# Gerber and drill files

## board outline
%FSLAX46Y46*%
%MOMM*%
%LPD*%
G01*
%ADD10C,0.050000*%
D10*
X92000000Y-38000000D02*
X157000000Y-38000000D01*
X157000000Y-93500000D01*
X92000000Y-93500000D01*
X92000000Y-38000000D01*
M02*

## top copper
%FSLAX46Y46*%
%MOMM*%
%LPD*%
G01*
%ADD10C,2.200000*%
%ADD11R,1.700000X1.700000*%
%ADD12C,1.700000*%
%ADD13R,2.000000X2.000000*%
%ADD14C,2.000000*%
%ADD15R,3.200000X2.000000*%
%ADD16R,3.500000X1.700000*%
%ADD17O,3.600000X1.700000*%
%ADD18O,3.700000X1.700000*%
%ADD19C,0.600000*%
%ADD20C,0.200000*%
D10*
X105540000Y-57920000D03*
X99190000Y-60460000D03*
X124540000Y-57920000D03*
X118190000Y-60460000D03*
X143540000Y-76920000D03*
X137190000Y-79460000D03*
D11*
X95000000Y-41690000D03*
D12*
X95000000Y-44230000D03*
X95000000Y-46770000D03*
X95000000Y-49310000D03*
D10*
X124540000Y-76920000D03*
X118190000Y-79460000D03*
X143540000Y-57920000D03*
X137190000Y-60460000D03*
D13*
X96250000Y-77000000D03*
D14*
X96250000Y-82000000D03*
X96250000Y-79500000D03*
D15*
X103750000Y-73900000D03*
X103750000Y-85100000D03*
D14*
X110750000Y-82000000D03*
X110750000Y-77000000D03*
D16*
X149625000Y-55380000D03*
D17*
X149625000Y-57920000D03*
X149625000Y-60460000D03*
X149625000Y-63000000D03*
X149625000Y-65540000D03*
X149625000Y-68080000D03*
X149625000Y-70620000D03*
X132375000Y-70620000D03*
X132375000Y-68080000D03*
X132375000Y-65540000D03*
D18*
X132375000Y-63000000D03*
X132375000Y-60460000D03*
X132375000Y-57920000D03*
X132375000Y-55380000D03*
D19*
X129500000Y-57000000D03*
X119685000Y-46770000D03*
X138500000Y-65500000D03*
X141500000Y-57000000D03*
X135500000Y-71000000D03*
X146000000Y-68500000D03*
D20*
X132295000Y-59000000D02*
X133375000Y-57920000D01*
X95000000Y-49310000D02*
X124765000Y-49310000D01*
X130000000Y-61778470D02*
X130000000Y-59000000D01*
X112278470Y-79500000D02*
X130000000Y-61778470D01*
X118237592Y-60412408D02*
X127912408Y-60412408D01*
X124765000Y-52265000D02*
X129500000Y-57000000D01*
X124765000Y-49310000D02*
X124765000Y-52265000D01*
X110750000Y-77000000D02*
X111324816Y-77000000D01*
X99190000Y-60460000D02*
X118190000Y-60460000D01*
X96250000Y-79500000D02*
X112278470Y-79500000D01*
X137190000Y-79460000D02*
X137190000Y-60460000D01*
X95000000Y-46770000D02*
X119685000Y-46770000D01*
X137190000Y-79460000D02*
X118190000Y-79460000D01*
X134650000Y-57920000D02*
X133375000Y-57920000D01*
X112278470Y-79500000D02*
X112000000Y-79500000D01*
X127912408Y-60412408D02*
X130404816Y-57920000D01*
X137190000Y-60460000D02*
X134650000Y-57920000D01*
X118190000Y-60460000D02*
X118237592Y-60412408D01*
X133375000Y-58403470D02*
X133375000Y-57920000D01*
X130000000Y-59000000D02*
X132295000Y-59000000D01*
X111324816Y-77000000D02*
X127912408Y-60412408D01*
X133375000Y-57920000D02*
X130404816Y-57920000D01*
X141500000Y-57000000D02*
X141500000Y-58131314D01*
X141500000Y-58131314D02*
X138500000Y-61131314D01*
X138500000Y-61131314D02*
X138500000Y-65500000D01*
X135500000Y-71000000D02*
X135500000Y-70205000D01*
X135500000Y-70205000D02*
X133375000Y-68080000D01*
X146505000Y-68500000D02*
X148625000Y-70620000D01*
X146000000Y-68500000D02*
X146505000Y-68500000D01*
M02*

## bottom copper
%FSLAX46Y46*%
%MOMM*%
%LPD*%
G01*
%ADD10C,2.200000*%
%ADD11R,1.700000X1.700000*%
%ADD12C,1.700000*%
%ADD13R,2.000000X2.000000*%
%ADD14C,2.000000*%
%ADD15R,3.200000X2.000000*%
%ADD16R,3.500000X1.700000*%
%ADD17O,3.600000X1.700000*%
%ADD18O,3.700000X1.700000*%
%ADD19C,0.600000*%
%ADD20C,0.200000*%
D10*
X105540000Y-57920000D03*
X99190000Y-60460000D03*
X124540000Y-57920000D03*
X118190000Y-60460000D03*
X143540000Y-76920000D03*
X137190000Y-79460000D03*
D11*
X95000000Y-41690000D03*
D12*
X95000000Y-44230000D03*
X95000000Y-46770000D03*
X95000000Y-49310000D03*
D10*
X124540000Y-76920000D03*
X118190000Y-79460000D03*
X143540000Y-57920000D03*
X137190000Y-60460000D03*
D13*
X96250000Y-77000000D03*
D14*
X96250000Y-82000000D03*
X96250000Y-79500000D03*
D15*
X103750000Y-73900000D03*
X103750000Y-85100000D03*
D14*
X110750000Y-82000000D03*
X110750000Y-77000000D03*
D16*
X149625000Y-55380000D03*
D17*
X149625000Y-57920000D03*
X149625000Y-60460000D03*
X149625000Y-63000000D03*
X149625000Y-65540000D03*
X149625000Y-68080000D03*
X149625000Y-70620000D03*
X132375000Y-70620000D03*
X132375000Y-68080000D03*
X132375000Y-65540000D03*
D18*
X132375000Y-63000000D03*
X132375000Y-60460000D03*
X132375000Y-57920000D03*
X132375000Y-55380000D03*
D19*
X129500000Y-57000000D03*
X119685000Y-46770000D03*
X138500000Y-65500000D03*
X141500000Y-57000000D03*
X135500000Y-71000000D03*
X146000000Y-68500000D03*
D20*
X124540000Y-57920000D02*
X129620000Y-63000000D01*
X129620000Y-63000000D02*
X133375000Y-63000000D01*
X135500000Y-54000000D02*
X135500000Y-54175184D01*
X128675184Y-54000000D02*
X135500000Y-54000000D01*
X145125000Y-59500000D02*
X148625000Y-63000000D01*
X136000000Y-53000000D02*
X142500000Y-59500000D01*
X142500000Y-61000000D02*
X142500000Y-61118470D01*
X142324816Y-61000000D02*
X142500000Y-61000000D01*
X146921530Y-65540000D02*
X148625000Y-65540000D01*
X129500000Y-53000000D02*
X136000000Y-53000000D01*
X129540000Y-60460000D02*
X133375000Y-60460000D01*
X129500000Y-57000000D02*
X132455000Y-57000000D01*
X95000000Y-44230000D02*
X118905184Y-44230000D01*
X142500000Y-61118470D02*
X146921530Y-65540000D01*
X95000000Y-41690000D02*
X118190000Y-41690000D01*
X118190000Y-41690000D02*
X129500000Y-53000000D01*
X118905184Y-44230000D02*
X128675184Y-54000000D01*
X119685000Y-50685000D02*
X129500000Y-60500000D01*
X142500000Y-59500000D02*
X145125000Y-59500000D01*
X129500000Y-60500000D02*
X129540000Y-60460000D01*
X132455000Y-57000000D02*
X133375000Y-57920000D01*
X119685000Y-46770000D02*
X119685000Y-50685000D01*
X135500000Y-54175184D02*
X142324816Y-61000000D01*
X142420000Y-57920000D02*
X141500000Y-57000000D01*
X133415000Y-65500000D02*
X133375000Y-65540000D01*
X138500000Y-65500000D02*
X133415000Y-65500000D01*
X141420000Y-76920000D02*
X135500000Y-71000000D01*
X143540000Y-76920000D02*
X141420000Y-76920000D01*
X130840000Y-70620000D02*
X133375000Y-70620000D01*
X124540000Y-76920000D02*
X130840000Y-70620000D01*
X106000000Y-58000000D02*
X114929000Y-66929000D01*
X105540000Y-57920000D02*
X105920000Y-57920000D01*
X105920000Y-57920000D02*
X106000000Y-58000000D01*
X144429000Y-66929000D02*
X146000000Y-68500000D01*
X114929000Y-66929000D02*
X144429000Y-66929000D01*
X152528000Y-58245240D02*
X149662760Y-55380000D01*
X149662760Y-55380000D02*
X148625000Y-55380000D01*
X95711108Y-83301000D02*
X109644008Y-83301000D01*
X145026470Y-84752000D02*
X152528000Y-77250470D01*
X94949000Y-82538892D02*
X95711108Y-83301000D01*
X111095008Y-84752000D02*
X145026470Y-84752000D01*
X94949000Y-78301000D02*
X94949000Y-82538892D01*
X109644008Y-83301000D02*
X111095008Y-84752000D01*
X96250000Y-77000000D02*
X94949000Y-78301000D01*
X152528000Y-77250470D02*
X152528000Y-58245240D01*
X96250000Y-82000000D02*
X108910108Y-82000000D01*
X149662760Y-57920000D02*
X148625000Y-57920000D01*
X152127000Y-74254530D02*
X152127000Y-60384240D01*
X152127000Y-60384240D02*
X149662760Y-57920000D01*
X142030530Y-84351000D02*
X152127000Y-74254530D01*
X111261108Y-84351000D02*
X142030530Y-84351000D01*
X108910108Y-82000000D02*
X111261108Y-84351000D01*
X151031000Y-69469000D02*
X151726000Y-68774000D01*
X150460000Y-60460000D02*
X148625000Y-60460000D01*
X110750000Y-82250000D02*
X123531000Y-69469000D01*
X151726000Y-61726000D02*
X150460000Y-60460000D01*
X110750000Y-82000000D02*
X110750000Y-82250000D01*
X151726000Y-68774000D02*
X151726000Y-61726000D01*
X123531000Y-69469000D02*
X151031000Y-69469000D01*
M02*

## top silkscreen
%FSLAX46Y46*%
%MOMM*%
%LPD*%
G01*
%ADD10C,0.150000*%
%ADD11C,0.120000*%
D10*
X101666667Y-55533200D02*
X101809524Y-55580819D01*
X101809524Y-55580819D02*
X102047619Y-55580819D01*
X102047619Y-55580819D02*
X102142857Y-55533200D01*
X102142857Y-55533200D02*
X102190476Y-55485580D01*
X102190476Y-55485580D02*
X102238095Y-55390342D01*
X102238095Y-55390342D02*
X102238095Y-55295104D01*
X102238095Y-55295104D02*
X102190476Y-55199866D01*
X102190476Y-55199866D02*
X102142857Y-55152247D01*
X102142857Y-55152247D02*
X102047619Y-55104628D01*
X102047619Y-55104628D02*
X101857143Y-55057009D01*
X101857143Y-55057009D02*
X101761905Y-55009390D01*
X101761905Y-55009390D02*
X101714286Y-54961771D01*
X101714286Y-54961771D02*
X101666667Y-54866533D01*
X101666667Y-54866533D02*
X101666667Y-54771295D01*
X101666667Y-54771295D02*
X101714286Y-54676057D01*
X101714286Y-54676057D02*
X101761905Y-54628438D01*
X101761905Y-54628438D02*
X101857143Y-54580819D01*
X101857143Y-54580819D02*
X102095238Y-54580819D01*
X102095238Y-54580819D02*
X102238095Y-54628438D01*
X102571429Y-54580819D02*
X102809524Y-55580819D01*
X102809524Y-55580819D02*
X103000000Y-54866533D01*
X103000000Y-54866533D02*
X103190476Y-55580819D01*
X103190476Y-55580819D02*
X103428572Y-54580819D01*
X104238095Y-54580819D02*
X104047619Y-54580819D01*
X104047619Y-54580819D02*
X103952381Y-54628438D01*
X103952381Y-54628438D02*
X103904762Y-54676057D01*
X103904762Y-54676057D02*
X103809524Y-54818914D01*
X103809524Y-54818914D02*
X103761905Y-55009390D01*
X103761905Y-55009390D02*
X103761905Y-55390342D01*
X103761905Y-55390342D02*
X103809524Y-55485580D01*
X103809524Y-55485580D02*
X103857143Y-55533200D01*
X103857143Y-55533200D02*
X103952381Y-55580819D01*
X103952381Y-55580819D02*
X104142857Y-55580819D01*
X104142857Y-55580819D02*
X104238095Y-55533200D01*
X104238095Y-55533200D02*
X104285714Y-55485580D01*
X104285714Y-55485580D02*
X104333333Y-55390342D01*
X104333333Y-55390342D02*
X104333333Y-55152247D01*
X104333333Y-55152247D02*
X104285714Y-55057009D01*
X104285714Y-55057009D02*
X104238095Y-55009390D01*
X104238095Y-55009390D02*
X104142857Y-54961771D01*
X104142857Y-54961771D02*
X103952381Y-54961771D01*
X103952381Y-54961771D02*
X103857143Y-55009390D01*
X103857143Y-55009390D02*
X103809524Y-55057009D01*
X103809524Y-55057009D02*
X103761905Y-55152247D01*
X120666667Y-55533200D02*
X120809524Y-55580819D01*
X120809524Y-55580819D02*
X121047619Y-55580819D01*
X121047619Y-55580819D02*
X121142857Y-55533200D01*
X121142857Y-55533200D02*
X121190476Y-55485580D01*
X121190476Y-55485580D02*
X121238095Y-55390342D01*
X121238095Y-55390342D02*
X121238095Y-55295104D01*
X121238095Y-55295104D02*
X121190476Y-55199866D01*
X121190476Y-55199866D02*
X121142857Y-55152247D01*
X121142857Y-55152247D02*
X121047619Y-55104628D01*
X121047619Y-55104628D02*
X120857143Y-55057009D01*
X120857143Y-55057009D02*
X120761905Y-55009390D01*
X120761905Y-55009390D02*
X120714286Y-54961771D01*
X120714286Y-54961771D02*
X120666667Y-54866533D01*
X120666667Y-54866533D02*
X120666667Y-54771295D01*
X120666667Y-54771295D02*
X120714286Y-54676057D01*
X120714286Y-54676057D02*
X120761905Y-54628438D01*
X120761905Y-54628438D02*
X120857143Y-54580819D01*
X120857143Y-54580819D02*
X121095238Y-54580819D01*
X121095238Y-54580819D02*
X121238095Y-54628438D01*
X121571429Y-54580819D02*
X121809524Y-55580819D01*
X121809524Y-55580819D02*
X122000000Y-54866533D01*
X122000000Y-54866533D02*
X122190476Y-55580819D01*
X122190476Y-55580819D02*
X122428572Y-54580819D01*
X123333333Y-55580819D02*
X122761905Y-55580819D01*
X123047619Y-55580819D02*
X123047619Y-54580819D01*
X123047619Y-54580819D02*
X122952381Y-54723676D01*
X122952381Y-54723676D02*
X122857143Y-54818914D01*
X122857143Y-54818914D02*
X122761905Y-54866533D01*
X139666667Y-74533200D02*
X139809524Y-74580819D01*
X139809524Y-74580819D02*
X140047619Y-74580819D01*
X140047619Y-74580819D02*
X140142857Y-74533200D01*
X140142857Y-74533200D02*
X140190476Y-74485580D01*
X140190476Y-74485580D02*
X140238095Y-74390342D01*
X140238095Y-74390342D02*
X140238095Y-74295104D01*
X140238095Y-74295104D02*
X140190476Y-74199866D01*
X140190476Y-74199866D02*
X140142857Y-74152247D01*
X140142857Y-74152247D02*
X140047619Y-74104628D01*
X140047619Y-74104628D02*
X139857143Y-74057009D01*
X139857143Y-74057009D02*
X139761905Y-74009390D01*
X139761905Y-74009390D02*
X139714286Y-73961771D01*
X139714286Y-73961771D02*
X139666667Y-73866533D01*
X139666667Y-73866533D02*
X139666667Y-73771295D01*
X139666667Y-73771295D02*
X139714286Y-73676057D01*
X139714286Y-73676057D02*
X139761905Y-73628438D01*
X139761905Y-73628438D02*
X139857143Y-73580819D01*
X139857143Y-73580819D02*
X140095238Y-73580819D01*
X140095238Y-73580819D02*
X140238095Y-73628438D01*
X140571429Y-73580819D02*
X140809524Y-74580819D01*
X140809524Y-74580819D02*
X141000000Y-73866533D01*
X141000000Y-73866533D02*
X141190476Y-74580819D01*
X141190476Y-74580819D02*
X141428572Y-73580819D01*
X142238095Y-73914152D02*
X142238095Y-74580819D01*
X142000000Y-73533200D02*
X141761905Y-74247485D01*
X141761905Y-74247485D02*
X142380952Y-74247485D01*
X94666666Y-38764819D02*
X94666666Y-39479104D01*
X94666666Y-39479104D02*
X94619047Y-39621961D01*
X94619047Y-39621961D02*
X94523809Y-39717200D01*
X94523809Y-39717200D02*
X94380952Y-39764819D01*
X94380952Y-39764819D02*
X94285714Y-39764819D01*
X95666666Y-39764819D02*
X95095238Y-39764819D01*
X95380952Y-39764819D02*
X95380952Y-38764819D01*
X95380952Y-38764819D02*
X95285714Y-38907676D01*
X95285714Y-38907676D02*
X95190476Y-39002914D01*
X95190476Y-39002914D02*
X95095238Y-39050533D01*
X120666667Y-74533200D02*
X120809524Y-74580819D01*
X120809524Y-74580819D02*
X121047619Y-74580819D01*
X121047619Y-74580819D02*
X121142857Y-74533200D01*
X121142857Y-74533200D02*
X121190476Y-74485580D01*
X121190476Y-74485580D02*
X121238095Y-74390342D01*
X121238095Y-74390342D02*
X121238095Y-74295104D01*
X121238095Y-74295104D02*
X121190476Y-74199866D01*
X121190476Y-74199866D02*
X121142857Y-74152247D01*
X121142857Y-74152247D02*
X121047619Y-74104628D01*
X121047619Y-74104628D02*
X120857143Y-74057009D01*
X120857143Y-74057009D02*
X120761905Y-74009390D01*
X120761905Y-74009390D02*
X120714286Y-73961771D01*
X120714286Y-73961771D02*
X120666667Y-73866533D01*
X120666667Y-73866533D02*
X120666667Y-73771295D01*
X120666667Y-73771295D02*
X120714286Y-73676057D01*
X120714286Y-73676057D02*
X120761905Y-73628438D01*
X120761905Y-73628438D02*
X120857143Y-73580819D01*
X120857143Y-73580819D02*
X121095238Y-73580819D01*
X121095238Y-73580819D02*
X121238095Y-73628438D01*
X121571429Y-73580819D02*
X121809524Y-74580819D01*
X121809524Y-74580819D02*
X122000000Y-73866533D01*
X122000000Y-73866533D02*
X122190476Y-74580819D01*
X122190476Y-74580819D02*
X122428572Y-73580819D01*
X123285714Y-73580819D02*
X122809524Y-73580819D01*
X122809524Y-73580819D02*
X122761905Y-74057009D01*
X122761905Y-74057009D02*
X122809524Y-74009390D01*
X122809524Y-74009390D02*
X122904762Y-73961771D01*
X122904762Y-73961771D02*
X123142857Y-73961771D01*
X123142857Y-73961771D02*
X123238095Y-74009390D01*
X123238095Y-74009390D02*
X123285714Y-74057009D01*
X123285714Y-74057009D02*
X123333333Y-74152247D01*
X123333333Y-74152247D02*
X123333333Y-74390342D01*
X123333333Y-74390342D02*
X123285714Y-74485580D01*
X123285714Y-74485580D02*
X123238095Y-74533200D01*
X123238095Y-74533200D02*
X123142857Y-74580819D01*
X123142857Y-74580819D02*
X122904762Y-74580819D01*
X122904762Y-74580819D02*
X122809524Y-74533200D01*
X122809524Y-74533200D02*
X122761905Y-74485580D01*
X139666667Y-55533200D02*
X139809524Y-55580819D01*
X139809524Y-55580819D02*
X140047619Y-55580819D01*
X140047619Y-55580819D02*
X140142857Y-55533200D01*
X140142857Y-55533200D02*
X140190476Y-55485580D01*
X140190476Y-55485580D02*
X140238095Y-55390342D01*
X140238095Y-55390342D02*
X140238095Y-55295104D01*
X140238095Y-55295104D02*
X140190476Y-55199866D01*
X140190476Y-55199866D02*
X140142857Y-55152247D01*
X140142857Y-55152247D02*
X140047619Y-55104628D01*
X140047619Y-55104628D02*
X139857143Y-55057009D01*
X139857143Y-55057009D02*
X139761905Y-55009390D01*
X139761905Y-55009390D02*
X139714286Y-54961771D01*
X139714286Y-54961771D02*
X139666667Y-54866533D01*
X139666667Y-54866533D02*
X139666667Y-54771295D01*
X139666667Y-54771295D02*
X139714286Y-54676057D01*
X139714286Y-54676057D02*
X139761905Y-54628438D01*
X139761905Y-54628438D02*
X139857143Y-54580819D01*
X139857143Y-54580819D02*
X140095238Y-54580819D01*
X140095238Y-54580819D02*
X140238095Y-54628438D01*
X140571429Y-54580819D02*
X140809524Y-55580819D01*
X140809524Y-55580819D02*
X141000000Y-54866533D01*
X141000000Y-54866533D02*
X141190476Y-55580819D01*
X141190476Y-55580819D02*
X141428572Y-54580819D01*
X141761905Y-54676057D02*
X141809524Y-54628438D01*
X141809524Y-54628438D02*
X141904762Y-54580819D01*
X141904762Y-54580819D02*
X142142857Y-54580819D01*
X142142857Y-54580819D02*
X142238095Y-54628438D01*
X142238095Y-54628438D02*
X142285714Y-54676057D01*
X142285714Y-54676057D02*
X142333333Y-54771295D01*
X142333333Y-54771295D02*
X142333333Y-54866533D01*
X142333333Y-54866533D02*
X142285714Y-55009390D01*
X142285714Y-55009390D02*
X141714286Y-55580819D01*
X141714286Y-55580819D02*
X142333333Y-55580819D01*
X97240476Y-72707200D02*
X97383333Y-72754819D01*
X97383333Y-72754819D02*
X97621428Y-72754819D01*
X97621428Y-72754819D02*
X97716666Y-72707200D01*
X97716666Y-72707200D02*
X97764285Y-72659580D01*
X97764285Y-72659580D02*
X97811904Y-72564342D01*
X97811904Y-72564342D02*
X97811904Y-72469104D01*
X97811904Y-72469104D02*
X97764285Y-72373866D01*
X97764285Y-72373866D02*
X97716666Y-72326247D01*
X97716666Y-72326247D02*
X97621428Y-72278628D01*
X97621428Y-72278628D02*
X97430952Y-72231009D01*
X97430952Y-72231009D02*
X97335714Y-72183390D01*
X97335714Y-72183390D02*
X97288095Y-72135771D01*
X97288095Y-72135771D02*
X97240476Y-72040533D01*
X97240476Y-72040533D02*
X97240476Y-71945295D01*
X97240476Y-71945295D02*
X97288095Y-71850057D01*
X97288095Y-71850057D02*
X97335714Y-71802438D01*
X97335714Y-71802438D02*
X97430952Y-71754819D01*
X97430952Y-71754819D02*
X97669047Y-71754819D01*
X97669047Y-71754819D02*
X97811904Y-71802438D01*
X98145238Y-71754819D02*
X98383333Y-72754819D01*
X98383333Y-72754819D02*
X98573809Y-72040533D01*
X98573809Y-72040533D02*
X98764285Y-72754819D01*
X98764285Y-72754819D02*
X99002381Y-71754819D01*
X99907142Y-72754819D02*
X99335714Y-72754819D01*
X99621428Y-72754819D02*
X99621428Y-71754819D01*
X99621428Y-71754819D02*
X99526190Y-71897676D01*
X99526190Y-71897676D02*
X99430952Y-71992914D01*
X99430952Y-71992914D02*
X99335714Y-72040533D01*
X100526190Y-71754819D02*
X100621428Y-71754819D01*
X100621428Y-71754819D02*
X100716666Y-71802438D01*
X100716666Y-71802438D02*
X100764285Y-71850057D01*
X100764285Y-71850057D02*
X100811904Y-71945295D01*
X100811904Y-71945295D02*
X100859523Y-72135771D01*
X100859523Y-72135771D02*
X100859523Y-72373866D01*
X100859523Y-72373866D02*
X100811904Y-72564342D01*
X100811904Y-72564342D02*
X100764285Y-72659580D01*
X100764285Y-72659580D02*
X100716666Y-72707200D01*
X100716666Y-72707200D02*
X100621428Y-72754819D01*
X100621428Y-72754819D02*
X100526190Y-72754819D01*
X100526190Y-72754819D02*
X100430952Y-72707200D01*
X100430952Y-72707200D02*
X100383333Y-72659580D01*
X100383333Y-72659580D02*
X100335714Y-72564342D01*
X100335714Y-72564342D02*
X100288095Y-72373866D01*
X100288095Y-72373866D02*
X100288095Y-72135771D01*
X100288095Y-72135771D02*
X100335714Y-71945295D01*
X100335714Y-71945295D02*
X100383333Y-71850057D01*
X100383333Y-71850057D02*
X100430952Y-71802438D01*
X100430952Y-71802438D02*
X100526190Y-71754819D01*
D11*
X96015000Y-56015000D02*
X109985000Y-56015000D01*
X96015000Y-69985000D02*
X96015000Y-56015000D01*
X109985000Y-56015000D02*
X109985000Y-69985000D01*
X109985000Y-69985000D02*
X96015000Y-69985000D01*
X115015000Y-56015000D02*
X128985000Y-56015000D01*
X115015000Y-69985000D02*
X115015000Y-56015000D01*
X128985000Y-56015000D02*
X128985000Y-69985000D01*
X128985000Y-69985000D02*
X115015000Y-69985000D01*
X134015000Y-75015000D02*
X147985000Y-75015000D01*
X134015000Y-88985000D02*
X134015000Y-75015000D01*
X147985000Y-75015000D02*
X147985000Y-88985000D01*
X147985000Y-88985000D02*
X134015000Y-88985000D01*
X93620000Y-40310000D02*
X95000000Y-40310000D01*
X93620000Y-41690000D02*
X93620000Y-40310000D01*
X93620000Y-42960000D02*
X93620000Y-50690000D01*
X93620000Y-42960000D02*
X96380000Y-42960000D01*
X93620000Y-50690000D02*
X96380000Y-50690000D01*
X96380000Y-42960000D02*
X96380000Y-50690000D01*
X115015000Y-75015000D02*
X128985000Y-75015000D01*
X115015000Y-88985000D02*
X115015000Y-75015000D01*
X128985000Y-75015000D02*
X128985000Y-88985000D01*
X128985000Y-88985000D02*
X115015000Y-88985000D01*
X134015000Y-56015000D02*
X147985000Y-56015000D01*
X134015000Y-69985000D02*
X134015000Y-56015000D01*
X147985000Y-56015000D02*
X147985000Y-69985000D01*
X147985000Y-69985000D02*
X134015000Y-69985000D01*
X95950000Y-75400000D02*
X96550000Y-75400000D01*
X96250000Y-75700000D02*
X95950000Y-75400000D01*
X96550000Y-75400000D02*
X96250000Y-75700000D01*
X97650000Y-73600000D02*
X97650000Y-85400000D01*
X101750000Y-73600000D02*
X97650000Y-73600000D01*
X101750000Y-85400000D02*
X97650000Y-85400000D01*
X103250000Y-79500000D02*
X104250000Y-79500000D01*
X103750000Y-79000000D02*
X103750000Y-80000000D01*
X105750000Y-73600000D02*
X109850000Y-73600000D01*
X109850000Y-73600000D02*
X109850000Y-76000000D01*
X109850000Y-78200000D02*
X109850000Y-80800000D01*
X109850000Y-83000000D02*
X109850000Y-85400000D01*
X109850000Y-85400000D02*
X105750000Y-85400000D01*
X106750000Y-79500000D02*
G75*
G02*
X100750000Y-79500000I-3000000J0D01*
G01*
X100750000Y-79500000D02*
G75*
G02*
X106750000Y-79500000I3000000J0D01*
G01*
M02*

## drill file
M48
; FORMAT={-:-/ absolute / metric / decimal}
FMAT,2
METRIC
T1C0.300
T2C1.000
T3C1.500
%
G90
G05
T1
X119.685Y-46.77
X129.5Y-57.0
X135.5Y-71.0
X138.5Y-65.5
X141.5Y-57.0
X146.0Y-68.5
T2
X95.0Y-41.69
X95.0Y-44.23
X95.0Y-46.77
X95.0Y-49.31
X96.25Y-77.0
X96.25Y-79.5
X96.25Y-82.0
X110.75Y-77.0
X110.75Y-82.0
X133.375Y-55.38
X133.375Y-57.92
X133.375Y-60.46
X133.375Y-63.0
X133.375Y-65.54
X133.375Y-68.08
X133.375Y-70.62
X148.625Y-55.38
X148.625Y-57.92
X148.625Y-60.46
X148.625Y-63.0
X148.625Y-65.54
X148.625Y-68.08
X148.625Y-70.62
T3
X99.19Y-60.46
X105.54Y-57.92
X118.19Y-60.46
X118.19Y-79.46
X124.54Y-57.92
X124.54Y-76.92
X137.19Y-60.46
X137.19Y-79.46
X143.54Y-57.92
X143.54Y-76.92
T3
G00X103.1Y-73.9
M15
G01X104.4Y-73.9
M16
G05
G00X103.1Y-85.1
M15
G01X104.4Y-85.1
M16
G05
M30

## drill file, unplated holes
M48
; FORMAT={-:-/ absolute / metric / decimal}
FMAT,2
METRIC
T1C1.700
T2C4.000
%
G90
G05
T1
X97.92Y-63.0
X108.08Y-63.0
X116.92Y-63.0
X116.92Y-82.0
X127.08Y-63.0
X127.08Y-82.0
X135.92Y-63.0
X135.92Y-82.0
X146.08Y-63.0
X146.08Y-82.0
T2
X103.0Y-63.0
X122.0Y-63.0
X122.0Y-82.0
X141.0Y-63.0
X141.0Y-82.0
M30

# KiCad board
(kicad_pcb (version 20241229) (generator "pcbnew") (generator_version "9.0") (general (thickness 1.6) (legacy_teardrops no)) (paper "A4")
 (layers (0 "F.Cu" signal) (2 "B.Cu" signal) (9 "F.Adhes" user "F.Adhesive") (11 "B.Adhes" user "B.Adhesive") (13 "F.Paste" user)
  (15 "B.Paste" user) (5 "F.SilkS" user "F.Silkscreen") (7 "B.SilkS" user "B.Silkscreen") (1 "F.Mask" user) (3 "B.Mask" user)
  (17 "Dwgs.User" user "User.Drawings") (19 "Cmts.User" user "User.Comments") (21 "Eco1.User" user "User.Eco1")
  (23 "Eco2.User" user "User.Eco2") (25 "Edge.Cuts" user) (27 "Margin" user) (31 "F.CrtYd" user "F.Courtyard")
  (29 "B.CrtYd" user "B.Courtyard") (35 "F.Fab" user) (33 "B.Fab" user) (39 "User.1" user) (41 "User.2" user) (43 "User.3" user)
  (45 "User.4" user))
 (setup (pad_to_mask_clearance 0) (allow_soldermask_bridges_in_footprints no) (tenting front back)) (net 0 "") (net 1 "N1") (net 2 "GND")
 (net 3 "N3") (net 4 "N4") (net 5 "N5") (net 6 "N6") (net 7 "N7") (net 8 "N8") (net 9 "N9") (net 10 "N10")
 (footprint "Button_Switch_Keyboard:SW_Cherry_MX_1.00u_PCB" (layer "F.Cu") (at 105.54 57.92)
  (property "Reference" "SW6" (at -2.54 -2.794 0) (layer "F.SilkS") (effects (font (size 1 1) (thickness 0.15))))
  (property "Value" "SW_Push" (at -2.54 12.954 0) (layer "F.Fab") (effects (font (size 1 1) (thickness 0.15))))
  (fp_line (start -9.525 -1.905) (end 4.445 -1.905) (stroke (width 0.12) (type solid)) (layer "F.SilkS"))
  (fp_line (start -9.525 12.065) (end -9.525 -1.905) (stroke (width 0.12) (type solid)) (layer "F.SilkS"))
  (fp_line (start 4.445 -1.905) (end 4.445 12.065) (stroke (width 0.12) (type solid)) (layer "F.SilkS"))
  (fp_line (start 4.445 12.065) (end -9.525 12.065) (stroke (width 0.12) (type solid)) (layer "F.SilkS"))
  (pad "" np_thru_hole circle (at -7.62 5.08) (size 1.7 1.7) (drill 1.7) (layers "*.Cu" "*.Mask"))
  (pad "" np_thru_hole circle (at -2.54 5.08) (size 4 4) (drill 4) (layers "*.Cu" "*.Mask"))
  (pad "" np_thru_hole circle (at 2.54 5.08) (size 1.7 1.7) (drill 1.7) (layers "*.Cu" "*.Mask"))
  (pad "1" thru_hole circle (at 0 0) (size 2.2 2.2) (drill 1.5) (layers "*.Cu" "*.Mask") (remove_unused_layers no) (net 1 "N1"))
  (pad "2" thru_hole circle (at -6.35 2.54) (size 2.2 2.2) (drill 1.5) (layers "*.Cu" "*.Mask") (remove_unused_layers no) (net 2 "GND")))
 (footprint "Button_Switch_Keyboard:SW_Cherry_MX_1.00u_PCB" (layer "F.Cu") (at 124.54 57.92)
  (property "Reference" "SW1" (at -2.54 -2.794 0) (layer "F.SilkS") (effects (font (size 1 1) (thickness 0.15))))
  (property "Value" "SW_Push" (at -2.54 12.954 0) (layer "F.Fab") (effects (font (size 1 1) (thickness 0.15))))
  (fp_line (start -9.525 -1.905) (end 4.445 -1.905) (stroke (width 0.12) (type solid)) (layer "F.SilkS"))
  (fp_line (start -9.525 12.065) (end -9.525 -1.905) (stroke (width 0.12) (type solid)) (layer "F.SilkS"))
  (fp_line (start 4.445 -1.905) (end 4.445 12.065) (stroke (width 0.12) (type solid)) (layer "F.SilkS"))
  (fp_line (start 4.445 12.065) (end -9.525 12.065) (stroke (width 0.12) (type solid)) (layer "F.SilkS"))
  (pad "" np_thru_hole circle (at -7.62 5.08) (size 1.7 1.7) (drill 1.7) (layers "*.Cu" "*.Mask"))
  (pad "" np_thru_hole circle (at -2.54 5.08) (size 4 4) (drill 4) (layers "*.Cu" "*.Mask"))
  (pad "" np_thru_hole circle (at 2.54 5.08) (size 1.7 1.7) (drill 1.7) (layers "*.Cu" "*.Mask"))
  (pad "1" thru_hole circle (at 0 0) (size 2.2 2.2) (drill 1.5) (layers "*.Cu" "*.Mask") (remove_unused_layers no) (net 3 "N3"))
  (pad "2" thru_hole circle (at -6.35 2.54) (size 2.2 2.2) (drill 1.5) (layers "*.Cu" "*.Mask") (remove_unused_layers no) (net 2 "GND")))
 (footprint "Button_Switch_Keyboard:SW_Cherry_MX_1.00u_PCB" (layer "F.Cu") (at 143.54 76.92)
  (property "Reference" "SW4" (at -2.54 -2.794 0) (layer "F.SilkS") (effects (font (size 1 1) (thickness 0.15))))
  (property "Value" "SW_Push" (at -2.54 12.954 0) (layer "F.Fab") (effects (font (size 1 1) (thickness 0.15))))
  (fp_line (start -9.525 -1.905) (end 4.445 -1.905) (stroke (width 0.12) (type solid)) (layer "F.SilkS"))
  (fp_line (start -9.525 12.065) (end -9.525 -1.905) (stroke (width 0.12) (type solid)) (layer "F.SilkS"))
  (fp_line (start 4.445 -1.905) (end 4.445 12.065) (stroke (width 0.12) (type solid)) (layer "F.SilkS"))
  (fp_line (start 4.445 12.065) (end -9.525 12.065) (stroke (width 0.12) (type solid)) (layer "F.SilkS"))
  (pad "" np_thru_hole circle (at -7.62 5.08) (size 1.7 1.7) (drill 1.7) (layers "*.Cu" "*.Mask"))
  (pad "" np_thru_hole circle (at -2.54 5.08) (size 4 4) (drill 4) (layers "*.Cu" "*.Mask"))
  (pad "" np_thru_hole circle (at 2.54 5.08) (size 1.7 1.7) (drill 1.7) (layers "*.Cu" "*.Mask"))
  (pad "1" thru_hole circle (at 0 0) (size 2.2 2.2) (drill 1.5) (layers "*.Cu" "*.Mask") (remove_unused_layers no) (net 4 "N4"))
  (pad "2" thru_hole circle (at -6.35 2.54) (size 2.2 2.2) (drill 1.5) (layers "*.Cu" "*.Mask") (remove_unused_layers no) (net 2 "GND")))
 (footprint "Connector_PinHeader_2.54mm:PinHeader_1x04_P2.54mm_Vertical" (layer "F.Cu") (at 95 41.69)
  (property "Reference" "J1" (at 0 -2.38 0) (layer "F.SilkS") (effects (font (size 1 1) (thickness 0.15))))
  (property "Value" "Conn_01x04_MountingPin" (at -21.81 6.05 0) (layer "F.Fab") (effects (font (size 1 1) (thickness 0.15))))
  (fp_line (start -1.38 -1.38) (end 0 -1.38) (stroke (width 0.12) (type solid)) (layer "F.SilkS"))
  (fp_line (start -1.38 0) (end -1.38 -1.38) (stroke (width 0.12) (type solid)) (layer "F.SilkS"))
  (fp_line (start -1.38 1.27) (end -1.38 9) (stroke (width 0.12) (type solid)) (layer "F.SilkS"))
  (fp_line (start -1.38 1.27) (end 1.38 1.27) (stroke (width 0.12) (type solid)) (layer "F.SilkS"))
  (fp_line (start -1.38 9) (end 1.38 9) (stroke (width 0.12) (type solid)) (layer "F.SilkS"))
  (fp_line (start 1.38 1.27) (end 1.38 9) (stroke (width 0.12) (type solid)) (layer "F.SilkS"))
  (pad "1" thru_hole rect (at 0 0) (size 1.7 1.7) (drill 1) (layers "*.Cu" "*.Mask") (remove_unused_layers no) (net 2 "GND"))
  (pad "2" thru_hole circle (at 0 2.54) (size 1.7 1.7) (drill 1) (layers "*.Cu" "*.Mask") (remove_unused_layers no) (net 2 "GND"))
  (pad "3" thru_hole circle (at 0 5.08) (size 1.7 1.7) (drill 1) (layers "*.Cu" "*.Mask") (remove_unused_layers no) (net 2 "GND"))
  (pad "4" thru_hole circle (at 0 7.62) (size 1.7 1.7) (drill 1) (layers "*.Cu" "*.Mask") (remove_unused_layers no) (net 2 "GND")))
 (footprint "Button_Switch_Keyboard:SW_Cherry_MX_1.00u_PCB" (layer "F.Cu") (at 124.54 76.92)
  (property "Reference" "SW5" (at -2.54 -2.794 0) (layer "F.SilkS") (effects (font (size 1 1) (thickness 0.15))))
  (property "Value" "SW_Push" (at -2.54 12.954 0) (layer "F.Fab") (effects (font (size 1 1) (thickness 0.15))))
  (fp_line (start -9.525 -1.905) (end 4.445 -1.905) (stroke (width 0.12) (type solid)) (layer "F.SilkS"))
  (fp_line (start -9.525 12.065) (end -9.525 -1.905) (stroke (width 0.12) (type solid)) (layer "F.SilkS"))
  (fp_line (start 4.445 -1.905) (end 4.445 12.065) (stroke (width 0.12) (type solid)) (layer "F.SilkS"))
  (fp_line (start 4.445 12.065) (end -9.525 12.065) (stroke (width 0.12) (type solid)) (layer "F.SilkS"))
  (pad "" np_thru_hole circle (at -7.62 5.08) (size 1.7 1.7) (drill 1.7) (layers "*.Cu" "*.Mask"))
  (pad "" np_thru_hole circle (at -2.54 5.08) (size 4 4) (drill 4) (layers "*.Cu" "*.Mask"))
  (pad "" np_thru_hole circle (at 2.54 5.08) (size 1.7 1.7) (drill 1.7) (layers "*.Cu" "*.Mask"))
  (pad "1" thru_hole circle (at 0 0) (size 2.2 2.2) (drill 1.5) (layers "*.Cu" "*.Mask") (remove_unused_layers no) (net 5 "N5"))
  (pad "2" thru_hole circle (at -6.35 2.54) (size 2.2 2.2) (drill 1.5) (layers "*.Cu" "*.Mask") (remove_unused_layers no) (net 2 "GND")))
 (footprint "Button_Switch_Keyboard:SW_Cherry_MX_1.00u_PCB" (layer "F.Cu") (at 143.54 57.92)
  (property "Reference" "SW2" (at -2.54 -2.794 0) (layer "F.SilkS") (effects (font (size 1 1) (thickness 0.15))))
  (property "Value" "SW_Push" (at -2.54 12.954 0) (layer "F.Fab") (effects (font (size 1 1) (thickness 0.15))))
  (fp_line (start -9.525 -1.905) (end 4.445 -1.905) (stroke (width 0.12) (type solid)) (layer "F.SilkS"))
  (fp_line (start -9.525 12.065) (end -9.525 -1.905) (stroke (width 0.12) (type solid)) (layer "F.SilkS"))
  (fp_line (start 4.445 -1.905) (end 4.445 12.065) (stroke (width 0.12) (type solid)) (layer "F.SilkS"))
  (fp_line (start 4.445 12.065) (end -9.525 12.065) (stroke (width 0.12) (type solid)) (layer "F.SilkS"))
  (pad "" np_thru_hole circle (at -7.62 5.08) (size 1.7 1.7) (drill 1.7) (layers "*.Cu" "*.Mask"))
  (pad "" np_thru_hole circle (at -2.54 5.08) (size 4 4) (drill 4) (layers "*.Cu" "*.Mask"))
  (pad "" np_thru_hole circle (at 2.54 5.08) (size 1.7 1.7) (drill 1.7) (layers "*.Cu" "*.Mask"))
  (pad "1" thru_hole circle (at 0 0) (size 2.2 2.2) (drill 1.5) (layers "*.Cu" "*.Mask") (remove_unused_layers no) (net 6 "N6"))
  (pad "2" thru_hole circle (at -6.35 2.54) (size 2.2 2.2) (drill 1.5) (layers "*.Cu" "*.Mask") (remove_unused_layers no) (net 2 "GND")))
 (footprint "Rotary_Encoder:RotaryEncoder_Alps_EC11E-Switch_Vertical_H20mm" (layer "F.Cu") (at 96.25 77)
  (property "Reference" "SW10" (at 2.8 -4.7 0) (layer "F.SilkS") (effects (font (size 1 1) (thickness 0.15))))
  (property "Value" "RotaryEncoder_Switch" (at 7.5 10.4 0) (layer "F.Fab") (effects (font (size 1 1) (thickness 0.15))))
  (fp_line (start -0.3 -1.6) (end 0.3 -1.6) (stroke (width 0.12) (type solid)) (layer "F.SilkS"))
  (fp_line (start 0 -1.3) (end -0.3 -1.6) (stroke (width 0.12) (type solid)) (layer "F.SilkS"))
  (fp_line (start 0.3 -1.6) (end 0 -1.3) (stroke (width 0.12) (type solid)) (layer "F.SilkS"))
  (fp_line (start 1.4 -3.4) (end 1.4 8.4) (stroke (width 0.12) (type solid)) (layer "F.SilkS"))
  (fp_line (start 5.5 -3.4) (end 1.4 -3.4) (stroke (width 0.12) (type solid)) (layer "F.SilkS"))
  (fp_line (start 5.5 8.4) (end 1.4 8.4) (stroke (width 0.12) (type solid)) (layer "F.SilkS"))
  (fp_line (start 7 2.5) (end 8 2.5) (stroke (width 0.12) (type solid)) (layer "F.SilkS"))
  (fp_line (start 7.5 2) (end 7.5 3) (stroke (width 0.12) (type solid)) (layer "F.SilkS"))
  (fp_line (start 9.5 -3.4) (end 13.6 -3.4) (stroke (width 0.12) (type solid)) (layer "F.SilkS"))
  (fp_line (start 13.6 -3.4) (end 13.6 -1) (stroke (width 0.12) (type solid)) (layer "F.SilkS"))
  (fp_line (start 13.6 1.2) (end 13.6 3.8) (stroke (width 0.12) (type solid)) (layer "F.SilkS"))
  (fp_line (start 13.6 6) (end 13.6 8.4) (stroke (width 0.12) (type solid)) (layer "F.SilkS"))
  (fp_line (start 13.6 8.4) (end 9.5 8.4) (stroke (width 0.12) (type solid)) (layer "F.SilkS"))
  (fp_circle (center 7.5 2.5) (end 10.5 2.5) (stroke (width 0.12) (type solid)) (fill no) (layer "F.SilkS"))
  (pad "A" thru_hole rect (at 0 0) (size 2 2) (drill 1) (layers "*.Cu" "*.Mask") (remove_unused_layers no) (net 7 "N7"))
  (pad "B" thru_hole circle (at 0 5) (size 2 2) (drill 1) (layers "*.Cu" "*.Mask") (remove_unused_layers no) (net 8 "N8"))
  (pad "C" thru_hole circle (at 0 2.5) (size 2 2) (drill 1) (layers "*.Cu" "*.Mask") (remove_unused_layers no) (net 2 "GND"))
  (pad "MP" thru_hole rect (at 7.5 -3.1) (size 3.2 2) (drill oval 2.8 1.5) (layers "*.Cu" "*.Mask") (remove_unused_layers no))
  (pad "MP" thru_hole rect (at 7.5 8.1) (size 3.2 2) (drill oval 2.8 1.5) (layers "*.Cu" "*.Mask") (remove_unused_layers no))
  (pad "S1" thru_hole circle (at 14.5 5) (size 2 2) (drill 1) (layers "*.Cu" "*.Mask") (remove_unused_layers no) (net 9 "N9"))
  (pad "S2" thru_hole circle (at 14.5 0) (size 2 2) (drill 1) (layers "*.Cu" "*.Mask") (remove_unused_layers no) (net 2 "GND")))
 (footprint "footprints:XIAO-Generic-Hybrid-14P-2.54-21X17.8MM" (layer "B.Cu") (at 141 63 180)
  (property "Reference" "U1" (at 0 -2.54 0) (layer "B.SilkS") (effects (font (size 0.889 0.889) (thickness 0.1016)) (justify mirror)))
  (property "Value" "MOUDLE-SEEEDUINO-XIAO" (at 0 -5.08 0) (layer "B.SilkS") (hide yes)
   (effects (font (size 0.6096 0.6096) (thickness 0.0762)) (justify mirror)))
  (pad "1" thru_hole rect (at -7.625 7.62 180) (size 3.5 1.7) (drill 1 (offset -1 0)) (layers "*.Cu" "*.Mask") (remove_unused_layers no)
   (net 7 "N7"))
  (pad "2" thru_hole oval (at -7.625 5.08 180) (size 3.6 1.7) (drill 1 (offset -1 0)) (layers "*.Cu" "*.Mask") (remove_unused_layers no)
   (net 8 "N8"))
  (pad "3" thru_hole oval (at -7.625 2.54 180) (size 3.6 1.7) (drill 1 (offset -1 0)) (layers "*.Cu" "*.Mask") (remove_unused_layers no)
   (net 9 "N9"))
  (pad "4" thru_hole oval (at -7.625 0 180) (size 3.6 1.7) (drill 1 (offset -1 0)) (layers "*.Cu" "*.Mask") (remove_unused_layers no)
   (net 2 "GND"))
  (pad "5" thru_hole oval (at -7.625 -2.54 180) (size 3.6 1.7) (drill 1 (offset -1 0)) (layers "*.Cu" "*.Mask") (remove_unused_layers no)
   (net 2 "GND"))
  (pad "6" thru_hole oval (at -7.625 -5.08) (size 3.6 1.7) (drill 1 (offset 1 0)) (layers "*.Cu" "*.Mask") (remove_unused_layers no)
   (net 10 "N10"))
  (pad "7" thru_hole oval (at -7.625 -7.62 180) (size 3.6 1.7) (drill 1 (offset -1 0)) (layers "*.Cu" "*.Mask") (remove_unused_layers no)
   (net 1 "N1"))
  (pad "8" thru_hole oval (at 7.625 -7.62 180) (size 3.6 1.7) (drill 1 (offset 1 0)) (layers "*.Cu" "*.Mask") (remove_unused_layers no)
   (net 5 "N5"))
  (pad "9" thru_hole oval (at 7.625 -5.08 180) (size 3.6 1.7) (drill 1 (offset 1 0)) (layers "*.Cu" "*.Mask") (remove_unused_layers no)
   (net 4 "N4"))
  (pad "10" thru_hole oval (at 7.625 -2.54 180) (size 3.6 1.7) (drill 1 (offset 1 0)) (layers "*.Cu" "*.Mask") (remove_unused_layers no)
   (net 6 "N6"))
  (pad "11" thru_hole oval (at 7.625 0 180) (size 3.7 1.7) (drill 1 (offset 1 0)) (layers "*.Cu" "*.Mask") (remove_unused_layers no)
   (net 3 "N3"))
  (pad "12" thru_hole oval (at 7.625 2.54 180) (size 3.7 1.7) (drill 1 (offset 1 0)) (layers "*.Cu" "*.Mask") (remove_unused_layers no)
   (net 2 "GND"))
  (pad "13" thru_hole oval (at 7.625 5.08 180) (size 3.7 1.7) (drill 1 (offset 1 0)) (layers "*.Cu" "*.Mask") (remove_unused_layers no)
   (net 2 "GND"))
  (pad "14" thru_hole oval (at 7.625 7.62 180) (size 3.7 1.7) (drill 1 (offset 1 0)) (layers "*.Cu" "*.Mask") (remove_unused_layers no)
   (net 2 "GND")))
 (gr_rect (start 92 38) (end 157 93.5) (stroke (width 0.05) (type default)) (fill no) (layer "Edge.Cuts"))
 (segment (start 124.54 57.92) (end 129.62 63) (width 0.2) (layer "B.Cu") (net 3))
 (segment (start 129.62 63) (end 133.375 63) (width 0.2) (layer "B.Cu") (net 3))
 (segment (start 132.295 59) (end 133.375 57.92) (width 0.2) (layer "F.Cu") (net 2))
 (segment (start 95 49.31) (end 124.765 49.31) (width 0.2) (layer "F.Cu") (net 2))
 (segment (start 130 61.77847) (end 130 59) (width 0.2) (layer "F.Cu") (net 2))
 (segment (start 112.27847 79.5) (end 130 61.77847) (width 0.2) (layer "F.Cu") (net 2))
 (segment (start 118.237592 60.412408) (end 127.912408 60.412408) (width 0.2) (layer "F.Cu") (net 2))
 (segment (start 124.765 52.265) (end 129.5 57) (width 0.2) (layer "F.Cu") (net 2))
 (segment (start 124.765 49.31) (end 124.765 52.265) (width 0.2) (layer "F.Cu") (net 2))
 (segment (start 110.75 77) (end 111.324816 77) (width 0.2) (layer "F.Cu") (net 2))
 (segment (start 99.19 60.46) (end 118.19 60.46) (width 0.2) (layer "F.Cu") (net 2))
 (segment (start 96.25 79.5) (end 112.27847 79.5) (width 0.2) (layer "F.Cu") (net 2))
 (segment (start 137.19 79.46) (end 137.19 60.46) (width 0.2) (layer "F.Cu") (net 2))
 (segment (start 95 46.77) (end 119.685 46.77) (width 0.2) (layer "F.Cu") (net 2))
 (segment (start 137.19 79.46) (end 118.19 79.46) (width 0.2) (layer "F.Cu") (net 2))
 (segment (start 134.65 57.92) (end 133.375 57.92) (width 0.2) (layer "F.Cu") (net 2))
 (segment (start 112.27847 79.5) (end 112 79.5) (width 0.2) (layer "F.Cu") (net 2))
 (segment (start 127.912408 60.412408) (end 130.404816 57.92) (width 0.2) (layer "F.Cu") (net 2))
 (segment (start 137.19 60.46) (end 134.65 57.92) (width 0.2) (layer "F.Cu") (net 2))
 (segment (start 118.19 60.46) (end 118.237592 60.412408) (width 0.2) (layer "F.Cu") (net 2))
 (segment (start 133.375 58.40347) (end 133.375 57.92) (width 0.2) (layer "F.Cu") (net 2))
 (segment (start 130 59) (end 132.295 59) (width 0.2) (layer "F.Cu") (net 2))
 (segment (start 111.324816 77) (end 127.912408 60.412408) (width 0.2) (layer "F.Cu") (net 2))
 (segment (start 133.375 57.92) (end 130.404816 57.92) (width 0.2) (layer "F.Cu") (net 2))
 (via (at 129.5 57) (size 0.6) (drill 0.3) (layers "F.Cu" "B.Cu") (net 2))
 (via (at 119.685 46.77) (size 0.6) (drill 0.3) (layers "F.Cu" "B.Cu") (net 2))
 (segment (start 135.5 54) (end 135.5 54.175184) (width 0.2) (layer "B.Cu") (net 2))
 (segment (start 128.675184 54) (end 135.5 54) (width 0.2) (layer "B.Cu") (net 2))
 (segment (start 145.125 59.5) (end 148.625 63) (width 0.2) (layer "B.Cu") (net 2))
 (segment (start 136 53) (end 142.5 59.5) (width 0.2) (layer "B.Cu") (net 2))
 (segment (start 142.5 61) (end 142.5 61.11847) (width 0.2) (layer "B.Cu") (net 2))
 (segment (start 142.324816 61) (end 142.5 61) (width 0.2) (layer "B.Cu") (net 2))
 (segment (start 146.92153 65.54) (end 148.625 65.54) (width 0.2) (layer "B.Cu") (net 2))
 (segment (start 129.5 53) (end 136 53) (width 0.2) (layer "B.Cu") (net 2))
 (segment (start 129.54 60.46) (end 133.375 60.46) (width 0.2) (layer "B.Cu") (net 2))
 (segment (start 129.5 57) (end 132.455 57) (width 0.2) (layer "B.Cu") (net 2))
 (segment (start 95 44.23) (end 118.905184 44.23) (width 0.2) (layer "B.Cu") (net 2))
 (segment (start 142.5 61.11847) (end 146.92153 65.54) (width 0.2) (layer "B.Cu") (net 2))
 (segment (start 95 41.69) (end 118.19 41.69) (width 0.2) (layer "B.Cu") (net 2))
 (segment (start 118.19 41.69) (end 129.5 53) (width 0.2) (layer "B.Cu") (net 2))
 (segment (start 118.905184 44.23) (end 128.675184 54) (width 0.2) (layer "B.Cu") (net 2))
 (segment (start 119.685 50.685) (end 129.5 60.5) (width 0.2) (layer "B.Cu") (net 2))
 (segment (start 142.5 59.5) (end 145.125 59.5) (width 0.2) (layer "B.Cu") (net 2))
 (segment (start 129.5 60.5) (end 129.54 60.46) (width 0.2) (layer "B.Cu") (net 2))
 (segment (start 132.455 57) (end 133.375 57.92) (width 0.2) (layer "B.Cu") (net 2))
 (segment (start 119.685 46.77) (end 119.685 50.685) (width 0.2) (layer "B.Cu") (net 2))
 (segment (start 135.5 54.175184) (end 142.324816 61) (width 0.2) (layer "B.Cu") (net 2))
 (segment (start 141.5 57) (end 141.5 58.131314) (width 0.2) (layer "F.Cu") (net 6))
 (segment (start 141.5 58.131314) (end 138.5 61.131314) (width 0.2) (layer "F.Cu") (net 6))
 (segment (start 138.5 61.131314) (end 138.5 65.5) (width 0.2) (layer "F.Cu") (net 6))
 (via (at 138.5 65.5) (size 0.6) (drill 0.3) (layers "F.Cu" "B.Cu") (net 6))
 (via (at 141.5 57) (size 0.6) (drill 0.3) (layers "F.Cu" "B.Cu") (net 6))
 (segment (start 142.42 57.92) (end 141.5 57) (width 0.2) (layer "B.Cu") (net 6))
 (segment (start 133.415 65.5) (end 133.375 65.54) (width 0.2) (layer "B.Cu") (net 6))
 (segment (start 138.5 65.5) (end 133.415 65.5) (width 0.2) (layer "B.Cu") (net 6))
 (segment (start 135.5 71) (end 135.5 70.205) (width 0.2) (layer "F.Cu") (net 4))
 (segment (start 135.5 70.205) (end 133.375 68.08) (width 0.2) (layer "F.Cu") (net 4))
 (via (at 135.5 71) (size 0.6) (drill 0.3) (layers "F.Cu" "B.Cu") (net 4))
 (segment (start 141.42 76.92) (end 135.5 71) (width 0.2) (layer "B.Cu") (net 4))
 (segment (start 143.54 76.92) (end 141.42 76.92) (width 0.2) (layer "B.Cu") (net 4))
 (segment (start 130.84 70.62) (end 133.375 70.62) (width 0.2) (layer "B.Cu") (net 5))
 (segment (start 124.54 76.92) (end 130.84 70.62) (width 0.2) (layer "B.Cu") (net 5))
 (segment (start 146.505 68.5) (end 148.625 70.62) (width 0.2) (layer "F.Cu") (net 1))
 (segment (start 146 68.5) (end 146.505 68.5) (width 0.2) (layer "F.Cu") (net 1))
 (via (at 146 68.5) (size 0.6) (drill 0.3) (layers "F.Cu" "B.Cu") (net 1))
 (segment (start 106 58) (end 114.929 66.929) (width 0.2) (layer "B.Cu") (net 1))
 (segment (start 105.54 57.92) (end 105.92 57.92) (width 0.2) (layer "B.Cu") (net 1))
 (segment (start 105.92 57.92) (end 106 58) (width 0.2) (layer "B.Cu") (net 1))
 (segment (start 144.429 66.929) (end 146 68.5) (width 0.2) (layer "B.Cu") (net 1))
 (segment (start 114.929 66.929) (end 144.429 66.929) (width 0.2) (layer "B.Cu") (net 1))
 (segment (start 152.528 58.24524) (end 149.66276 55.38) (width 0.2) (layer "B.Cu") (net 7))
 (segment (start 149.66276 55.38) (end 148.625 55.38) (width 0.2) (layer "B.Cu") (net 7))
 (segment (start 95.711108 83.301) (end 109.644008 83.301) (width 0.2) (layer "B.Cu") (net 7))
 (segment (start 145.02647 84.752) (end 152.528 77.25047) (width 0.2) (layer "B.Cu") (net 7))
 (segment (start 94.949 82.538892) (end 95.711108 83.301) (width 0.2) (layer "B.Cu") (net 7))
 (segment (start 111.095008 84.752) (end 145.02647 84.752) (width 0.2) (layer "B.Cu") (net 7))
 (segment (start 94.949 78.301) (end 94.949 82.538892) (width 0.2) (layer "B.Cu") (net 7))
 (segment (start 109.644008 83.301) (end 111.095008 84.752) (width 0.2) (layer "B.Cu") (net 7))
 (segment (start 96.25 77) (end 94.949 78.301) (width 0.2) (layer "B.Cu") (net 7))
 (segment (start 152.528 77.25047) (end 152.528 58.24524) (width 0.2) (layer "B.Cu") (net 7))
 (segment (start 96.25 82) (end 108.910108 82) (width 0.2) (layer "B.Cu") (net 8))
 (segment (start 149.66276 57.92) (end 148.625 57.92) (width 0.2) (layer "B.Cu") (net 8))
 (segment (start 152.127 74.25453) (end 152.127 60.38424) (width 0.2) (layer "B.Cu") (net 8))
 (segment (start 152.127 60.38424) (end 149.66276 57.92) (width 0.2) (layer "B.Cu") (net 8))
 (segment (start 142.03053 84.351) (end 152.127 74.25453) (width 0.2) (layer "B.Cu") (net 8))
 (segment (start 111.261108 84.351) (end 142.03053 84.351) (width 0.2) (layer "B.Cu") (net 8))
 (segment (start 108.910108 82) (end 111.261108 84.351) (width 0.2) (layer "B.Cu") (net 8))
 (segment (start 151.031 69.469) (end 151.726 68.774) (width 0.2) (layer "B.Cu") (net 9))
 (segment (start 150.46 60.46) (end 148.625 60.46) (width 0.2) (layer "B.Cu") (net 9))
 (segment (start 110.75 82.25) (end 123.531 69.469) (width 0.2) (layer "B.Cu") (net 9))
 (segment (start 151.726 61.726) (end 150.46 60.46) (width 0.2) (layer "B.Cu") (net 9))
 (segment (start 110.75 82) (end 110.75 82.25) (width 0.2) (layer "B.Cu") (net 9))
 (segment (start 151.726 68.774) (end 151.726 61.726) (width 0.2) (layer "B.Cu") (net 9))
 (segment (start 123.531 69.469) (end 151.031 69.469) (width 0.2) (layer "B.Cu") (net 9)))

